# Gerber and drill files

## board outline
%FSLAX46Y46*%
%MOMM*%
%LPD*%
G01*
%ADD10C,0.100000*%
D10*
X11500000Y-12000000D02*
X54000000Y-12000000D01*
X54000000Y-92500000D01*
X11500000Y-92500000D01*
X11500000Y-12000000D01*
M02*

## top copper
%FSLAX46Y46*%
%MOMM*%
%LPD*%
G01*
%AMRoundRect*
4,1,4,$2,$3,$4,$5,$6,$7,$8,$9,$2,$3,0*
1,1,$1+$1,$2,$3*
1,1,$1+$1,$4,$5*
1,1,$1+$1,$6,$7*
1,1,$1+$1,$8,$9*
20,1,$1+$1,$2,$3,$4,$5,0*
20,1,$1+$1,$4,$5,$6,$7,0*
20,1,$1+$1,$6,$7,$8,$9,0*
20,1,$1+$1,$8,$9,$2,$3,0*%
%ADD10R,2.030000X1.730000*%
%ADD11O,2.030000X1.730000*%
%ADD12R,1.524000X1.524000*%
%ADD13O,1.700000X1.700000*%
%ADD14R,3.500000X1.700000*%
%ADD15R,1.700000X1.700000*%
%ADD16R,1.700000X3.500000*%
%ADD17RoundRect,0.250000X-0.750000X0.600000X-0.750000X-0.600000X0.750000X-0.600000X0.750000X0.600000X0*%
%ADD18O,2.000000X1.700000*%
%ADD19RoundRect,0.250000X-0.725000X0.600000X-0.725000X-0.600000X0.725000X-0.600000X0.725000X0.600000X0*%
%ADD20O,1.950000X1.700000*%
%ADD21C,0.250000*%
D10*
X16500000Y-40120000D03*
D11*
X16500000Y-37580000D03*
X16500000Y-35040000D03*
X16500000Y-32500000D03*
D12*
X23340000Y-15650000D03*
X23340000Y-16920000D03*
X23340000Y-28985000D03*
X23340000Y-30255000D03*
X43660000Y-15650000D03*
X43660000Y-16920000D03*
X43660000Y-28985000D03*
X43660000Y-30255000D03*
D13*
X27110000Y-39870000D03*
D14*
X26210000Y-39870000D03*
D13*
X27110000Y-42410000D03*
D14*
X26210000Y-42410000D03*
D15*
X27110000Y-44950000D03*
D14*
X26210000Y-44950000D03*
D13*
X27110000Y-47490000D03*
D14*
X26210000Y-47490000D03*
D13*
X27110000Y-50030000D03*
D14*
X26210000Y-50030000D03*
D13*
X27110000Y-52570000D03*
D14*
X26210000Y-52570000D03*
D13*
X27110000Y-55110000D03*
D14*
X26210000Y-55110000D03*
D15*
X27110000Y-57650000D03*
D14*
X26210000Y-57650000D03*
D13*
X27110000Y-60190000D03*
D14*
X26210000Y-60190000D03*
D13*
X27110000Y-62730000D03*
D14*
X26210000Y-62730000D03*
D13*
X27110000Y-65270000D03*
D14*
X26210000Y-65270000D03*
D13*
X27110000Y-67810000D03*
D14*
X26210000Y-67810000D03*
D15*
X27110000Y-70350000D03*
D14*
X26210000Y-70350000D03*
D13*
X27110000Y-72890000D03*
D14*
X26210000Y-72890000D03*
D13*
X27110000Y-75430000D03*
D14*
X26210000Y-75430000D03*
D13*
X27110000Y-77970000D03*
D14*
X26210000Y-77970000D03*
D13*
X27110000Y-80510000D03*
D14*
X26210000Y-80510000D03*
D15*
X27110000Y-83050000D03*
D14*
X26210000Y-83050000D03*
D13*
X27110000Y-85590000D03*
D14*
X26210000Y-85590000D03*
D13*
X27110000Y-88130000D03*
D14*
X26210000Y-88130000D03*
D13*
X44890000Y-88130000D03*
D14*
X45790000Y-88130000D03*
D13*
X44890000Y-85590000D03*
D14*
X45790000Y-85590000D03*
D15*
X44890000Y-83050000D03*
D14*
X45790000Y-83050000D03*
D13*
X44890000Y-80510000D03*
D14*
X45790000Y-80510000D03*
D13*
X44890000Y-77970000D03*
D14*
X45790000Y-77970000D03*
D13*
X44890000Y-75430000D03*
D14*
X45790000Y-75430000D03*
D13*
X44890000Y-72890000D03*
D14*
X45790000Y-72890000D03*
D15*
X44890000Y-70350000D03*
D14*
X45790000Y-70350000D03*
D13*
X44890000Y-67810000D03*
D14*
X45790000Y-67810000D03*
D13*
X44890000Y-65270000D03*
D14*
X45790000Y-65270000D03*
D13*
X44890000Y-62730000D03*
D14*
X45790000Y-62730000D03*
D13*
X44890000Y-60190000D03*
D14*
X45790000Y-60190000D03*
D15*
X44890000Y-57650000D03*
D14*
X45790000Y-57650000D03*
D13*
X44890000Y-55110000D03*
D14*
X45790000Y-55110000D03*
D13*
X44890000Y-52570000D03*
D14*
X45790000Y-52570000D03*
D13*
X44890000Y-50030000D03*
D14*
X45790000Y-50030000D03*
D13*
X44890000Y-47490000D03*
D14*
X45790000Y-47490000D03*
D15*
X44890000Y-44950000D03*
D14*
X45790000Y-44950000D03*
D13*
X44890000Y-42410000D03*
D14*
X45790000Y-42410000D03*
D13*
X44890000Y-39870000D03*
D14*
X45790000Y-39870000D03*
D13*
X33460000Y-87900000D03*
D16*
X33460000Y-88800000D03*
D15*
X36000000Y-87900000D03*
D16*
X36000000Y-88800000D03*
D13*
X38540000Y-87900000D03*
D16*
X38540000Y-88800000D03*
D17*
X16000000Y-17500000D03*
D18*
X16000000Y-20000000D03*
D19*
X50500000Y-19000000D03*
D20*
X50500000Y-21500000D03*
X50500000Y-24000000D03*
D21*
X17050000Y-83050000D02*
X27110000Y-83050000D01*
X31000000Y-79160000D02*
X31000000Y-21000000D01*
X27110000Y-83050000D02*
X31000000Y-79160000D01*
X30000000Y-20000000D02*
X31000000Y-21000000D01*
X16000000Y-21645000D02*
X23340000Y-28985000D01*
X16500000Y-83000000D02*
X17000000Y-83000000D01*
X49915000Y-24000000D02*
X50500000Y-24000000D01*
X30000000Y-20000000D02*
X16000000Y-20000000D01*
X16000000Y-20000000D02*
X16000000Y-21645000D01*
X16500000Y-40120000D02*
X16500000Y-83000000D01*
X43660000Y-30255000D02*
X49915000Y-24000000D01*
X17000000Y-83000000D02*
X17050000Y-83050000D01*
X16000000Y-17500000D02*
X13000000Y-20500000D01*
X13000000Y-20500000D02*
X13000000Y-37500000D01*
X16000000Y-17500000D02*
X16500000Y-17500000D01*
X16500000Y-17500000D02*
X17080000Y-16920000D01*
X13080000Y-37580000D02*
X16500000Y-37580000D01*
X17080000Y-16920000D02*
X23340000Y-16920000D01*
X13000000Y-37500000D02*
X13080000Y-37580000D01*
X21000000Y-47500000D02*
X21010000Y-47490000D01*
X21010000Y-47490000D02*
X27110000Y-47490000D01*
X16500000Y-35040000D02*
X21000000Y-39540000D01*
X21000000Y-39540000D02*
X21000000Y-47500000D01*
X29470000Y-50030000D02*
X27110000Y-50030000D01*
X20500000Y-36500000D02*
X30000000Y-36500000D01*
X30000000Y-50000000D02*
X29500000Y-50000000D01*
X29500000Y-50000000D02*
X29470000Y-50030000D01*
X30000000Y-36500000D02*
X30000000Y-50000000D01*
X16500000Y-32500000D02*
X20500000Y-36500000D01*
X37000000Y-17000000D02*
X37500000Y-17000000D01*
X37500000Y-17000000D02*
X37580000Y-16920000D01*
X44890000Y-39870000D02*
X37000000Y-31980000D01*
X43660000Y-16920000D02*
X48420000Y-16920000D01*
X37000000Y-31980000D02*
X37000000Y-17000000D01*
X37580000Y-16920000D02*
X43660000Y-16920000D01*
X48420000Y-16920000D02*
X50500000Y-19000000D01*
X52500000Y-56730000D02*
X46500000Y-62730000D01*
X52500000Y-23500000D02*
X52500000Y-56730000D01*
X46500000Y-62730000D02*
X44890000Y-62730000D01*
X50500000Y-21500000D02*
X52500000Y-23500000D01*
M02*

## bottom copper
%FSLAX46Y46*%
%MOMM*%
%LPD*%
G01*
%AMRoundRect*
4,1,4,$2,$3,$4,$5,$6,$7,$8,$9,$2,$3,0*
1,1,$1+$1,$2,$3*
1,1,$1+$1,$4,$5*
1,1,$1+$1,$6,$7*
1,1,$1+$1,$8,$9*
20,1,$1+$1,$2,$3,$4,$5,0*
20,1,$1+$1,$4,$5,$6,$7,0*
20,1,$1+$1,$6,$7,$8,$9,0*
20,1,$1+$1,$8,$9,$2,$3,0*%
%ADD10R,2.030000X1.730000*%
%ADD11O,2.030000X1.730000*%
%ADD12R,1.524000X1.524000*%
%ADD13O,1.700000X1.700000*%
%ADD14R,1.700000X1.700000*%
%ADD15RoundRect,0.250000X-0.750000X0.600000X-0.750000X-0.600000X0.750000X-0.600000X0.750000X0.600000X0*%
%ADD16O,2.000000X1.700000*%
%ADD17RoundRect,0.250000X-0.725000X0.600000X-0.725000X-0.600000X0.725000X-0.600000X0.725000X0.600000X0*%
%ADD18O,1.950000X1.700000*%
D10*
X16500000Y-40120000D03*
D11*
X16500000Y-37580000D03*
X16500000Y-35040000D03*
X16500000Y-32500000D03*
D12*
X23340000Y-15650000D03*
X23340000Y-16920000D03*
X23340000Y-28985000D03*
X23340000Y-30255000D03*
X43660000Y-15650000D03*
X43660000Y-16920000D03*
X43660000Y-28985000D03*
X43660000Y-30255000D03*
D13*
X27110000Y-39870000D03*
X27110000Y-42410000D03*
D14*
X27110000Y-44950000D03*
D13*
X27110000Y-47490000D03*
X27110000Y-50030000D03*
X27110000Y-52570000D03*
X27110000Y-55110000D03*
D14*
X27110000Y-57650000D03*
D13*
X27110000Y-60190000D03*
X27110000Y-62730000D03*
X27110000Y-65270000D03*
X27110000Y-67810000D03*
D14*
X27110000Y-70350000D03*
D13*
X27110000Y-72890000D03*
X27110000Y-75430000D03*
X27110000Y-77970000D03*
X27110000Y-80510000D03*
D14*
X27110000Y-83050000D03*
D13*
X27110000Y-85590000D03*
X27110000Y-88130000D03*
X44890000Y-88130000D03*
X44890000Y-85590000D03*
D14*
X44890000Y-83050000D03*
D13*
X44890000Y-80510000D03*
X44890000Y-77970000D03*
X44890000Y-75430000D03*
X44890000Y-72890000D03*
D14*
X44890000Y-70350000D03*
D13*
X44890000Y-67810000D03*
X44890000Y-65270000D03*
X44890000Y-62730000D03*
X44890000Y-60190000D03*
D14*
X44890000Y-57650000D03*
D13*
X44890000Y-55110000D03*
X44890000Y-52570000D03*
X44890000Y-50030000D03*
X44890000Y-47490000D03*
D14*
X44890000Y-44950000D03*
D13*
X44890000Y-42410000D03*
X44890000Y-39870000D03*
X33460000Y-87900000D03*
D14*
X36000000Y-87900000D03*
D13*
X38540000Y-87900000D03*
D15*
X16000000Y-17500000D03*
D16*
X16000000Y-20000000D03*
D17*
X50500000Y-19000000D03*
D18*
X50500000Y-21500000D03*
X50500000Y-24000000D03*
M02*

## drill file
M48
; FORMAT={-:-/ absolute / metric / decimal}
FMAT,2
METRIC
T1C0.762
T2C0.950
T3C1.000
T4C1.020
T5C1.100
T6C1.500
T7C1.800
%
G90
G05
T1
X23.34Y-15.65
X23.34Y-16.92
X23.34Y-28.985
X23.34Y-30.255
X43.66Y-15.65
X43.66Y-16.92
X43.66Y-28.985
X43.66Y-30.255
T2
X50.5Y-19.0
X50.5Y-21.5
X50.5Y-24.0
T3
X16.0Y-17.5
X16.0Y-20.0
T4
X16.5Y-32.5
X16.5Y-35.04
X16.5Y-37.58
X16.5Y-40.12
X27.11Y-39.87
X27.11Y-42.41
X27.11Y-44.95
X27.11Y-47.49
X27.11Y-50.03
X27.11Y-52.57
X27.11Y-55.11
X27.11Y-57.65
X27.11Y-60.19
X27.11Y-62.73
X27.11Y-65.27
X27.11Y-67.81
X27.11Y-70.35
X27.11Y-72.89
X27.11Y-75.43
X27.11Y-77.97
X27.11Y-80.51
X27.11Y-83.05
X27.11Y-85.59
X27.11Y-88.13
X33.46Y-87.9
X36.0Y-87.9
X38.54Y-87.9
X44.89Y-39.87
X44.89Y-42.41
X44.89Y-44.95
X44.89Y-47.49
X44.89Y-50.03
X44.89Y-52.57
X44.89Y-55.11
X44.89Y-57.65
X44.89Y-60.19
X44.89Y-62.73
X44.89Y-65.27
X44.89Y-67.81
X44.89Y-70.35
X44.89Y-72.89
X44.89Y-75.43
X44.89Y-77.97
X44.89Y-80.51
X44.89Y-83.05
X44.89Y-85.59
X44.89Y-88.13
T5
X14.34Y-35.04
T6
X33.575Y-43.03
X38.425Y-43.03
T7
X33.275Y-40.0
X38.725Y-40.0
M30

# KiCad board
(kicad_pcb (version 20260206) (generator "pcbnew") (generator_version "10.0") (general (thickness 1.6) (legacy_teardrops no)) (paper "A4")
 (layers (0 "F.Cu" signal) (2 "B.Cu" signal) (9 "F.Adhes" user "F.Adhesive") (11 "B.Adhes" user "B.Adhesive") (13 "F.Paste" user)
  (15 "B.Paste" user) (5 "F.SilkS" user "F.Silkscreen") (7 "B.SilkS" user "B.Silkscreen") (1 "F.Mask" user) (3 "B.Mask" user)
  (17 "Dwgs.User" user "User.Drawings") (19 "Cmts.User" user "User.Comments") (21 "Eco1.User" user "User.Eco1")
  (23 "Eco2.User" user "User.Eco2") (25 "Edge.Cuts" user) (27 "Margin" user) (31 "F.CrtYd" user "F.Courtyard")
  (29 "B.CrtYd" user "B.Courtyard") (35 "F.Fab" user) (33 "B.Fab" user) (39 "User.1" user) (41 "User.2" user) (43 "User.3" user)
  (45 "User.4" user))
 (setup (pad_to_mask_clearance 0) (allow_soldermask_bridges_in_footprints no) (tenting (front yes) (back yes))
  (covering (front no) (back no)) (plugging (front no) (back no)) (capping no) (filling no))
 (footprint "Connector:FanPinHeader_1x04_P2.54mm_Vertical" (layer "F.Cu") (at 16.5 40.12 90)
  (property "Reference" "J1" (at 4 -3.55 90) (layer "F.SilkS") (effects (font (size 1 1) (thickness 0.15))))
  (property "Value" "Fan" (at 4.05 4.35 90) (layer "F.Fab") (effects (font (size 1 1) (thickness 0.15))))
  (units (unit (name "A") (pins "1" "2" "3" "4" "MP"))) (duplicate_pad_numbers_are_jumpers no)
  (pad "" np_thru_hole circle (at 5.08 -2.16 180) (size 1.1 1.1) (drill 1.1) (layers "*.Cu" "*.Mask"))
  (pad "1" thru_hole rect (at 0 0 180) (size 2.03 1.73) (drill 1.02) (layers "*.Cu" "*.Mask") (remove_unused_layers no) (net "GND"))
  (pad "2" thru_hole oval (at 2.54 0 180) (size 2.03 1.73) (drill 1.02) (layers "*.Cu" "*.Mask") (remove_unused_layers no) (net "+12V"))
  (pad "3" thru_hole oval (at 5.08 0 180) (size 2.03 1.73) (drill 1.02) (layers "*.Cu" "*.Mask") (remove_unused_layers no)
   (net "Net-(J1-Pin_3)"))
  (pad "4" thru_hole oval (at 7.62 0 180) (size 2.03 1.73) (drill 1.02) (layers "*.Cu" "*.Mask") (remove_unused_layers no)
   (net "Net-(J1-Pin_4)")))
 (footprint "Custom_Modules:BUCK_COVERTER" (layer "F.Cu") (at 33.5 22)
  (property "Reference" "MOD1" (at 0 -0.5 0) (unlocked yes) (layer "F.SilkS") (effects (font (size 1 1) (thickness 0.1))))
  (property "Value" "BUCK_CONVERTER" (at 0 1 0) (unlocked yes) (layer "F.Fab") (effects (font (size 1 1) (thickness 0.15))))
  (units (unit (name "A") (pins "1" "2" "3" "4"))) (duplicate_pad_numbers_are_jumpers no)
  (pad "1" thru_hole rect (at -10.16 -6.35) (size 1.524 1.524) (drill 0.762) (layers "*.Cu" "*.Mask") (remove_unused_layers no) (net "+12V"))
  (pad "1" thru_hole rect (at -10.16 -5.08) (size 1.524 1.524) (drill 0.762) (layers "*.Cu" "*.Mask") (remove_unused_layers no) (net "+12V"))
  (pad "2" thru_hole rect (at -10.16 6.985) (size 1.524 1.524) (drill 0.762) (layers "*.Cu" "*.Mask") (remove_unused_layers no) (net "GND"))
  (pad "2" thru_hole rect (at -10.16 8.255) (size 1.524 1.524) (drill 0.762) (layers "*.Cu" "*.Mask") (remove_unused_layers no) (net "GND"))
  (pad "3" thru_hole rect (at 10.16 -6.35) (size 1.524 1.524) (drill 0.762) (layers "*.Cu" "*.Mask") (remove_unused_layers no) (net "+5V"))
  (pad "3" thru_hole rect (at 10.16 -5.08) (size 1.524 1.524) (drill 0.762) (layers "*.Cu" "*.Mask") (remove_unused_layers no) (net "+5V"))
  (pad "4" thru_hole rect (at 10.16 6.985) (size 1.524 1.524) (drill 0.762) (layers "*.Cu" "*.Mask") (remove_unused_layers no) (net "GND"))
  (pad "4" thru_hole rect (at 10.16 8.255) (size 1.524 1.524) (drill 0.762) (layers "*.Cu" "*.Mask") (remove_unused_layers no) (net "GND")))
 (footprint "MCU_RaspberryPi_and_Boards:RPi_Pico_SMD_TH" (layer "F.Cu") (at 36 64)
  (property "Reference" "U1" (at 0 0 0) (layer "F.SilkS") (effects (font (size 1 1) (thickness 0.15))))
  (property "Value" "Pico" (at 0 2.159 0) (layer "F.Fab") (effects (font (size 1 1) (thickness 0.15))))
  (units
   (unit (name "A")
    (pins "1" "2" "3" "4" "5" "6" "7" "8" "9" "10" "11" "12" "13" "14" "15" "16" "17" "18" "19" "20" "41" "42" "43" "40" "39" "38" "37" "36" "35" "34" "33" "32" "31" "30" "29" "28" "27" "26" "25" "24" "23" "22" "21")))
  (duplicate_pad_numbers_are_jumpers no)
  (pad "" np_thru_hole oval (at -2.725 -24) (size 1.8 1.8) (drill 1.8) (layers "*.Cu" "*.Mask"))
  (pad "" np_thru_hole oval (at -2.425 -20.97) (size 1.5 1.5) (drill 1.5) (layers "*.Cu" "*.Mask"))
  (pad "" np_thru_hole oval (at 2.425 -20.97) (size 1.5 1.5) (drill 1.5) (layers "*.Cu" "*.Mask"))
  (pad "" np_thru_hole oval (at 2.725 -24) (size 1.8 1.8) (drill 1.8) (layers "*.Cu" "*.Mask"))
  (pad "1" thru_hole oval (at -8.89 -24.13) (size 1.7 1.7) (drill 1.02) (layers "*.Cu" "*.Mask") (remove_unused_layers no)
   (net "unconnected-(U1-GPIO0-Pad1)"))
  (pad "1" smd rect (at -8.89 -24.13) (size 3.5 1.7) (drill (offset -0.9 0)) (layers "F.Cu" "F.Mask") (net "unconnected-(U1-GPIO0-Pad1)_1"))
  (pad "2" thru_hole oval (at -8.89 -21.59) (size 1.7 1.7) (drill 1.02) (layers "*.Cu" "*.Mask") (remove_unused_layers no)
   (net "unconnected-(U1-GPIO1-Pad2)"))
  (pad "2" smd rect (at -8.89 -21.59) (size 3.5 1.7) (drill (offset -0.9 0)) (layers "F.Cu" "F.Mask") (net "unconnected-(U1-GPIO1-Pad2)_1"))
  (pad "3" thru_hole rect (at -8.89 -19.05) (size 1.7 1.7) (drill 1.02) (layers "*.Cu" "*.Mask") (remove_unused_layers no) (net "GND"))
  (pad "3" smd rect (at -8.89 -19.05) (size 3.5 1.7) (drill (offset -0.9 0)) (layers "F.Cu" "F.Mask") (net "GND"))
  (pad "4" thru_hole oval (at -8.89 -16.51) (size 1.7 1.7) (drill 1.02) (layers "*.Cu" "*.Mask") (remove_unused_layers no)
   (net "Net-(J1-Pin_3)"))
  (pad "4" smd rect (at -8.89 -16.51) (size 3.5 1.7) (drill (offset -0.9 0)) (layers "F.Cu" "F.Mask") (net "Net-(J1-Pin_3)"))
  (pad "5" thru_hole oval (at -8.89 -13.97) (size 1.7 1.7) (drill 1.02) (layers "*.Cu" "*.Mask") (remove_unused_layers no)
   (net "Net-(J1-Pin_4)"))
  (pad "5" smd rect (at -8.89 -13.97) (size 3.5 1.7) (drill (offset -0.9 0)) (layers "F.Cu" "F.Mask") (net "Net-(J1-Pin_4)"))
  (pad "6" thru_hole oval (at -8.89 -11.43) (size 1.7 1.7) (drill 1.02) (layers "*.Cu" "*.Mask") (remove_unused_layers no)
   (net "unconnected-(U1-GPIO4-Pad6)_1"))
  (pad "6" smd rect (at -8.89 -11.43) (size 3.5 1.7) (drill (offset -0.9 0)) (layers "F.Cu" "F.Mask") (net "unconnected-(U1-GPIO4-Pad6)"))
  (pad "7" thru_hole oval (at -8.89 -8.89) (size 1.7 1.7) (drill 1.02) (layers "*.Cu" "*.Mask") (remove_unused_layers no)
   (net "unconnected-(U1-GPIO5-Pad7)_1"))
  (pad "7" smd rect (at -8.89 -8.89) (size 3.5 1.7) (drill (offset -0.9 0)) (layers "F.Cu" "F.Mask") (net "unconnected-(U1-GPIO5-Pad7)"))
  (pad "8" thru_hole rect (at -8.89 -6.35) (size 1.7 1.7) (drill 1.02) (layers "*.Cu" "*.Mask") (remove_unused_layers no)
   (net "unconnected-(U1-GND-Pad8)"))
  (pad "8" smd rect (at -8.89 -6.35) (size 3.5 1.7) (drill (offset -0.9 0)) (layers "F.Cu" "F.Mask") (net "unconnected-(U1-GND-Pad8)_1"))
  (pad "9" thru_hole oval (at -8.89 -3.81) (size 1.7 1.7) (drill 1.02) (layers "*.Cu" "*.Mask") (remove_unused_layers no)
   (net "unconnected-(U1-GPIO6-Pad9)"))
  (pad "9" smd rect (at -8.89 -3.81) (size 3.5 1.7) (drill (offset -0.9 0)) (layers "F.Cu" "F.Mask") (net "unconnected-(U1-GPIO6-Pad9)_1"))
  (pad "10" thru_hole oval (at -8.89 -1.27) (size 1.7 1.7) (drill 1.02) (layers "*.Cu" "*.Mask") (remove_unused_layers no)
   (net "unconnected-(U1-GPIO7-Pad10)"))
  (pad "10" smd rect (at -8.89 -1.27) (size 3.5 1.7) (drill (offset -0.9 0)) (layers "F.Cu" "F.Mask") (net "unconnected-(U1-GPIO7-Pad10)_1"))
  (pad "11" thru_hole oval (at -8.89 1.27) (size 1.7 1.7) (drill 1.02) (layers "*.Cu" "*.Mask") (remove_unused_layers no)
   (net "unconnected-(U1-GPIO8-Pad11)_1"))
  (pad "11" smd rect (at -8.89 1.27) (size 3.5 1.7) (drill (offset -0.9 0)) (layers "F.Cu" "F.Mask") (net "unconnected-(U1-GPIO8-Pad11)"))
  (pad "12" thru_hole oval (at -8.89 3.81) (size 1.7 1.7) (drill 1.02) (layers "*.Cu" "*.Mask") (remove_unused_layers no)
   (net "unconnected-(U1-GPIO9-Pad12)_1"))
  (pad "12" smd rect (at -8.89 3.81) (size 3.5 1.7) (drill (offset -0.9 0)) (layers "F.Cu" "F.Mask") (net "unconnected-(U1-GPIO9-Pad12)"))
  (pad "13" thru_hole rect (at -8.89 6.35) (size 1.7 1.7) (drill 1.02) (layers "*.Cu" "*.Mask") (remove_unused_layers no)
   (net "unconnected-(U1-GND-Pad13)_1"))
  (pad "13" smd rect (at -8.89 6.35) (size 3.5 1.7) (drill (offset -0.9 0)) (layers "F.Cu" "F.Mask") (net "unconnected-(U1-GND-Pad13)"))
  (pad "14" thru_hole oval (at -8.89 8.89) (size 1.7 1.7) (drill 1.02) (layers "*.Cu" "*.Mask") (remove_unused_layers no)
   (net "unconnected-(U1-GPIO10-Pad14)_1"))
  (pad "14" smd rect (at -8.89 8.89) (size 3.5 1.7) (drill (offset -0.9 0)) (layers "F.Cu" "F.Mask") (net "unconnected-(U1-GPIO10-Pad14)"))
  (pad "15" thru_hole oval (at -8.89 11.43) (size 1.7 1.7) (drill 1.02) (layers "*.Cu" "*.Mask") (remove_unused_layers no)
   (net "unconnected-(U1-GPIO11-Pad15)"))
  (pad "15" smd rect (at -8.89 11.43) (size 3.5 1.7) (drill (offset -0.9 0)) (layers "F.Cu" "F.Mask")
   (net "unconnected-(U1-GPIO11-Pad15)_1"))
  (pad "16" thru_hole oval (at -8.89 13.97) (size 1.7 1.7) (drill 1.02) (layers "*.Cu" "*.Mask") (remove_unused_layers no)
   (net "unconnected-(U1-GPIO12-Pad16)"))
  (pad "16" smd rect (at -8.89 13.97) (size 3.5 1.7) (drill (offset -0.9 0)) (layers "F.Cu" "F.Mask")
   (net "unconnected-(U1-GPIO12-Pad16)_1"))
  (pad "17" thru_hole oval (at -8.89 16.51) (size 1.7 1.7) (drill 1.02) (layers "*.Cu" "*.Mask") (remove_unused_layers no)
   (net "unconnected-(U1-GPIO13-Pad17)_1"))
  (pad "17" smd rect (at -8.89 16.51) (size 3.5 1.7) (drill (offset -0.9 0)) (layers "F.Cu" "F.Mask") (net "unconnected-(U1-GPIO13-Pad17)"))
  (pad "18" thru_hole rect (at -8.89 19.05) (size 1.7 1.7) (drill 1.02) (layers "*.Cu" "*.Mask") (remove_unused_layers no) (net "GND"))
  (pad "18" smd rect (at -8.89 19.05) (size 3.5 1.7) (drill (offset -0.9 0)) (layers "F.Cu" "F.Mask") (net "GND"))
  (pad "19" thru_hole oval (at -8.89 21.59) (size 1.7 1.7) (drill 1.02) (layers "*.Cu" "*.Mask") (remove_unused_layers no)
   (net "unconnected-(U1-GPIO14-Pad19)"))
  (pad "19" smd rect (at -8.89 21.59) (size 3.5 1.7) (drill (offset -0.9 0)) (layers "F.Cu" "F.Mask")
   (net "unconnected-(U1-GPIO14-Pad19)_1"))
  (pad "20" thru_hole oval (at -8.89 24.13) (size 1.7 1.7) (drill 1.02) (layers "*.Cu" "*.Mask") (remove_unused_layers no)
   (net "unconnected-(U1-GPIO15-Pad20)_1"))
  (pad "20" smd rect (at -8.89 24.13) (size 3.5 1.7) (drill (offset -0.9 0)) (layers "F.Cu" "F.Mask") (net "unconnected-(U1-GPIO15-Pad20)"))
  (pad "21" thru_hole oval (at 8.89 24.13) (size 1.7 1.7) (drill 1.02) (layers "*.Cu" "*.Mask") (remove_unused_layers no)
   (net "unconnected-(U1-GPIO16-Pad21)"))
  (pad "21" smd rect (at 8.89 24.13) (size 3.5 1.7) (drill (offset 0.9 0)) (layers "F.Cu" "F.Mask") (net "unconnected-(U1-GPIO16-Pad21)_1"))
  (pad "22" thru_hole oval (at 8.89 21.59) (size 1.7 1.7) (drill 1.02) (layers "*.Cu" "*.Mask") (remove_unused_layers no)
   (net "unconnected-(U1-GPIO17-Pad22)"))
  (pad "22" smd rect (at 8.89 21.59) (size 3.5 1.7) (drill (offset 0.9 0)) (layers "F.Cu" "F.Mask") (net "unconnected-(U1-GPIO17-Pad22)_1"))
  (pad "23" thru_hole rect (at 8.89 19.05) (size 1.7 1.7) (drill 1.02) (layers "*.Cu" "*.Mask") (remove_unused_layers no)
   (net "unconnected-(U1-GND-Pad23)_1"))
  (pad "23" smd rect (at 8.89 19.05) (size 3.5 1.7) (drill (offset 0.9 0)) (layers "F.Cu" "F.Mask") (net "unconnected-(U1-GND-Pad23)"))
  (pad "24" thru_hole oval (at 8.89 16.51) (size 1.7 1.7) (drill 1.02) (layers "*.Cu" "*.Mask") (remove_unused_layers no)
   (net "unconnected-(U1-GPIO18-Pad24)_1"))
  (pad "24" smd rect (at 8.89 16.51) (size 3.5 1.7) (drill (offset 0.9 0)) (layers "F.Cu" "F.Mask") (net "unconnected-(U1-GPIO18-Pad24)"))
  (pad "25" thru_hole oval (at 8.89 13.97) (size 1.7 1.7) (drill 1.02) (layers "*.Cu" "*.Mask") (remove_unused_layers no)
   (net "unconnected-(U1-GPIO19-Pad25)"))
  (pad "25" smd rect (at 8.89 13.97) (size 3.5 1.7) (drill (offset 0.9 0)) (layers "F.Cu" "F.Mask") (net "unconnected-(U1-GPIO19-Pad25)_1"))
  (pad "26" thru_hole oval (at 8.89 11.43) (size 1.7 1.7) (drill 1.02) (layers "*.Cu" "*.Mask") (remove_unused_layers no)
   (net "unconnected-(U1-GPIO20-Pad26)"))
  (pad "26" smd rect (at 8.89 11.43) (size 3.5 1.7) (drill (offset 0.9 0)) (layers "F.Cu" "F.Mask") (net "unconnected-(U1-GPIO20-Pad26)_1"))
  (pad "27" thru_hole oval (at 8.89 8.89) (size 1.7 1.7) (drill 1.02) (layers "*.Cu" "*.Mask") (remove_unused_layers no)
   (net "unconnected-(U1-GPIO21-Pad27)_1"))
  (pad "27" smd rect (at 8.89 8.89) (size 3.5 1.7) (drill (offset 0.9 0)) (layers "F.Cu" "F.Mask") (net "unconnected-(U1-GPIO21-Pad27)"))
  (pad "28" thru_hole rect (at 8.89 6.35) (size 1.7 1.7) (drill 1.02) (layers "*.Cu" "*.Mask") (remove_unused_layers no)
   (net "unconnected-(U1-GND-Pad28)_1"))
  (pad "28" smd rect (at 8.89 6.35) (size 3.5 1.7) (drill (offset 0.9 0)) (layers "F.Cu" "F.Mask") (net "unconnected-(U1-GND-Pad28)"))
  (pad "29" thru_hole oval (at 8.89 3.81) (size 1.7 1.7) (drill 1.02) (layers "*.Cu" "*.Mask") (remove_unused_layers no)
   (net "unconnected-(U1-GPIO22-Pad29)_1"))
  (pad "29" smd rect (at 8.89 3.81) (size 3.5 1.7) (drill (offset 0.9 0)) (layers "F.Cu" "F.Mask") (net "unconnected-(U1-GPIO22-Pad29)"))
  (pad "30" thru_hole oval (at 8.89 1.27) (size 1.7 1.7) (drill 1.02) (layers "*.Cu" "*.Mask") (remove_unused_layers no)
   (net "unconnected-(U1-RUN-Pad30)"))
  (pad "30" smd rect (at 8.89 1.27) (size 3.5 1.7) (drill (offset 0.9 0)) (layers "F.Cu" "F.Mask") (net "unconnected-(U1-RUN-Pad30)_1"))
  (pad "31" thru_hole oval (at 8.89 -1.27) (size 1.7 1.7) (drill 1.02) (layers "*.Cu" "*.Mask") (remove_unused_layers no)
   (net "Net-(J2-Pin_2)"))
  (pad "31" smd rect (at 8.89 -1.27) (size 3.5 1.7) (drill (offset 0.9 0)) (layers "F.Cu" "F.Mask") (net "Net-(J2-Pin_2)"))
  (pad "32" thru_hole oval (at 8.89 -3.81) (size 1.7 1.7) (drill 1.02) (layers "*.Cu" "*.Mask") (remove_unused_layers no)
   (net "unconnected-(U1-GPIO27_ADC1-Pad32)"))
  (pad "32" smd rect (at 8.89 -3.81) (size 3.5 1.7) (drill (offset 0.9 0)) (layers "F.Cu" "F.Mask")
   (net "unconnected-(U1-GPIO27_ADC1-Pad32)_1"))
  (pad "33" thru_hole rect (at 8.89 -6.35) (size 1.7 1.7) (drill 1.02) (layers "*.Cu" "*.Mask") (remove_unused_layers no)
   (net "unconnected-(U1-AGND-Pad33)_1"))
  (pad "33" smd rect (at 8.89 -6.35) (size 3.5 1.7) (drill (offset 0.9 0)) (layers "F.Cu" "F.Mask") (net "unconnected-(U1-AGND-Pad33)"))
  (pad "34" thru_hole oval (at 8.89 -8.89) (size 1.7 1.7) (drill 1.02) (layers "*.Cu" "*.Mask") (remove_unused_layers no)
   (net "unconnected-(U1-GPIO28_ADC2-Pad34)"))
  (pad "34" smd rect (at 8.89 -8.89) (size 3.5 1.7) (drill (offset 0.9 0)) (layers "F.Cu" "F.Mask")
   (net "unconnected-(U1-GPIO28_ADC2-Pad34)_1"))
  (pad "35" thru_hole oval (at 8.89 -11.43) (size 1.7 1.7) (drill 1.02) (layers "*.Cu" "*.Mask") (remove_unused_layers no)
   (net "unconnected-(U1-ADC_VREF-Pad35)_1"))
  (pad "35" smd rect (at 8.89 -11.43) (size 3.5 1.7) (drill (offset 0.9 0)) (layers "F.Cu" "F.Mask") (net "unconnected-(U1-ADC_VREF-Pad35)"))
  (pad "36" thru_hole oval (at 8.89 -13.97) (size 1.7 1.7) (drill 1.02) (layers "*.Cu" "*.Mask") (remove_unused_layers no)
   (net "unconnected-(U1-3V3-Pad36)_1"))
  (pad "36" smd rect (at 8.89 -13.97) (size 3.5 1.7) (drill (offset 0.9 0)) (layers "F.Cu" "F.Mask") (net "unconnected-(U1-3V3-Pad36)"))
  (pad "37" thru_hole oval (at 8.89 -16.51) (size 1.7 1.7) (drill 1.02) (layers "*.Cu" "*.Mask") (remove_unused_layers no)
   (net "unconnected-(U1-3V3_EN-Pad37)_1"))
  (pad "37" smd rect (at 8.89 -16.51) (size 3.5 1.7) (drill (offset 0.9 0)) (layers "F.Cu" "F.Mask") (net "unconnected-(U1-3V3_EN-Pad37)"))
  (pad "38" thru_hole rect (at 8.89 -19.05) (size 1.7 1.7) (drill 1.02) (layers "*.Cu" "*.Mask") (remove_unused_layers no)
   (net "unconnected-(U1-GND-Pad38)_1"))
  (pad "38" smd rect (at 8.89 -19.05) (size 3.5 1.7) (drill (offset 0.9 0)) (layers "F.Cu" "F.Mask") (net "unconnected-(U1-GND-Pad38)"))
  (pad "39" thru_hole oval (at 8.89 -21.59) (size 1.7 1.7) (drill 1.02) (layers "*.Cu" "*.Mask") (remove_unused_layers no)
   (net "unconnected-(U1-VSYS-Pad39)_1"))
  (pad "39" smd rect (at 8.89 -21.59) (size 3.5 1.7) (drill (offset 0.9 0)) (layers "F.Cu" "F.Mask") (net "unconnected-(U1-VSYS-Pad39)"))
  (pad "40" thru_hole oval (at 8.89 -24.13) (size 1.7 1.7) (drill 1.02) (layers "*.Cu" "*.Mask") (remove_unused_layers no) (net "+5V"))
  (pad "40" smd rect (at 8.89 -24.13) (size 3.5 1.7) (drill (offset 0.9 0)) (layers "F.Cu" "F.Mask") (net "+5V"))
  (pad "41" thru_hole oval (at -2.54 23.9) (size 1.7 1.7) (drill 1.02) (layers "*.Cu" "*.Mask") (remove_unused_layers no)
   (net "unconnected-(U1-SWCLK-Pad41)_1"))
  (pad "41" smd rect (at -2.54 23.9 90) (size 3.5 1.7) (drill (offset -0.9 0)) (layers "F.Cu" "F.Mask") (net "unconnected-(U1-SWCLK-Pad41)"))
  (pad "42" thru_hole rect (at 0 23.9) (size 1.7 1.7) (drill 1.02) (layers "*.Cu" "*.Mask") (remove_unused_layers no)
   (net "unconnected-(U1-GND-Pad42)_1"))
  (pad "42" smd rect (at 0 23.9 90) (size 3.5 1.7) (drill (offset -0.9 0)) (layers "F.Cu" "F.Mask") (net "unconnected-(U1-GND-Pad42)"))
  (pad "43" thru_hole oval (at 2.54 23.9) (size 1.7 1.7) (drill 1.02) (layers "*.Cu" "*.Mask") (remove_unused_layers no)
   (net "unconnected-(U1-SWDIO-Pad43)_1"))
  (pad "43" smd rect (at 2.54 23.9 90) (size 3.5 1.7) (drill (offset -0.9 0)) (layers "F.Cu" "F.Mask") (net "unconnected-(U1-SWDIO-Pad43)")))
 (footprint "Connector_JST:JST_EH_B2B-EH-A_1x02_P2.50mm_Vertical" (layer "F.Cu") (at 16 17.5 -90)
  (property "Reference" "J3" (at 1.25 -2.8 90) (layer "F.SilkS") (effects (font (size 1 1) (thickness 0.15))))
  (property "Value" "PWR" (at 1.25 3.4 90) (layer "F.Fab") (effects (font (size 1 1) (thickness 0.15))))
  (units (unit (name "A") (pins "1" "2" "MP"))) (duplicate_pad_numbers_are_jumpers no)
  (pad "1" thru_hole roundrect (at 0 0 270) (size 1.7 2) (drill 1) (layers "*.Cu" "*.Mask") (remove_unused_layers no)
   (roundrect_rratio 0.147059) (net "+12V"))
  (pad "2" thru_hole oval (at 2.5 0 270) (size 1.7 2) (drill 1) (layers "*.Cu" "*.Mask") (remove_unused_layers no) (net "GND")))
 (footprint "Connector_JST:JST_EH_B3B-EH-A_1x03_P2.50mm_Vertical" (layer "F.Cu") (at 50.5 19 -90)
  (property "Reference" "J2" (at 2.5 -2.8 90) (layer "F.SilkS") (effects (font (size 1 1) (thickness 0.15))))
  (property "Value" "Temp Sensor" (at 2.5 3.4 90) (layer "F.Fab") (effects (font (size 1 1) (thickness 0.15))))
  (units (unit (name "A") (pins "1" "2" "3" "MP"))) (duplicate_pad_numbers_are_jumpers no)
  (pad "1" thru_hole roundrect (at 0 0 270) (size 1.7 1.95) (drill 0.95) (layers "*.Cu" "*.Mask") (remove_unused_layers no)
   (roundrect_rratio 0.147059) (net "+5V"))
  (pad "2" thru_hole oval (at 2.5 0 270) (size 1.7 1.95) (drill 0.95) (layers "*.Cu" "*.Mask") (remove_unused_layers no)
   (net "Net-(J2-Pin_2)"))
  (pad "3" thru_hole oval (at 5 0 270) (size 1.7 1.95) (drill 0.95) (layers "*.Cu" "*.Mask") (remove_unused_layers no) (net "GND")))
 (gr_rect (start 11.5 12) (end 54 92.5) (stroke (width 0.1) (type default)) (fill no) (layer "Edge.Cuts"))
 (segment (start 17.05 83.05) (end 27.11 83.05) (width 0.25) (layer "F.Cu") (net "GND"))
 (segment (start 31 79.16) (end 31 21) (width 0.25) (layer "F.Cu") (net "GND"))
 (segment (start 27.11 83.05) (end 31 79.16) (width 0.25) (layer "F.Cu") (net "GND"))
 (segment (start 30 20) (end 31 21) (width 0.25) (layer "F.Cu") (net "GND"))
 (segment (start 16 21.645) (end 23.34 28.985) (width 0.25) (layer "F.Cu") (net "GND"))
 (segment (start 16.5 83) (end 17 83) (width 0.25) (layer "F.Cu") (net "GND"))
 (segment (start 49.915 24) (end 50.5 24) (width 0.25) (layer "F.Cu") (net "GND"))
 (segment (start 30 20) (end 16 20) (width 0.25) (layer "F.Cu") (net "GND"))
 (segment (start 16 20) (end 16 21.645) (width 0.25) (layer "F.Cu") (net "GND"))
 (segment (start 16.5 40.12) (end 16.5 83) (width 0.25) (layer "F.Cu") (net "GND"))
 (segment (start 43.66 30.255) (end 49.915 24) (width 0.25) (layer "F.Cu") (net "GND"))
 (segment (start 17 83) (end 17.05 83.05) (width 0.25) (layer "F.Cu") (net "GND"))
 (segment (start 16 17.5) (end 13 20.5) (width 0.25) (layer "F.Cu") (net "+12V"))
 (segment (start 13 20.5) (end 13 37.5) (width 0.25) (layer "F.Cu") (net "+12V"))
 (segment (start 16 17.5) (end 16.5 17.5) (width 0.25) (layer "F.Cu") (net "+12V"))
 (segment (start 16.5 17.5) (end 17.08 16.92) (width 0.25) (layer "F.Cu") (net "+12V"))
 (segment (start 13.08 37.58) (end 16.5 37.58) (width 0.25) (layer "F.Cu") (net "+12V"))
 (segment (start 17.08 16.92) (end 23.34 16.92) (width 0.25) (layer "F.Cu") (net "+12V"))
 (segment (start 13 37.5) (end 13.08 37.58) (width 0.25) (layer "F.Cu") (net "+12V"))
 (segment (start 21 47.5) (end 21.01 47.49) (width 0.25) (layer "F.Cu") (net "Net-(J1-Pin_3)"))
 (segment (start 21.01 47.49) (end 27.11 47.49) (width 0.25) (layer "F.Cu") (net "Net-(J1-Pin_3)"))
 (segment (start 16.5 35.04) (end 21 39.54) (width 0.25) (layer "F.Cu") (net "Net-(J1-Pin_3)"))
 (segment (start 21 39.54) (end 21 47.5) (width 0.25) (layer "F.Cu") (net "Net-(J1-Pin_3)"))
 (segment (start 29.47 50.03) (end 27.11 50.03) (width 0.25) (layer "F.Cu") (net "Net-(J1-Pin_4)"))
 (segment (start 20.5 36.5) (end 30 36.5) (width 0.25) (layer "F.Cu") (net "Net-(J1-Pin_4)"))
 (segment (start 30 50) (end 29.5 50) (width 0.25) (layer "F.Cu") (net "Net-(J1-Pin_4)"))
 (segment (start 29.5 50) (end 29.47 50.03) (width 0.25) (layer "F.Cu") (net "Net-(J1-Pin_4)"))
 (segment (start 30 36.5) (end 30 50) (width 0.25) (layer "F.Cu") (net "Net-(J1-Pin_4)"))
 (segment (start 16.5 32.5) (end 20.5 36.5) (width 0.25) (layer "F.Cu") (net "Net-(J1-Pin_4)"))
 (segment (start 37 17) (end 37.5 17) (width 0.25) (layer "F.Cu") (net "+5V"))
 (segment (start 37.5 17) (end 37.58 16.92) (width 0.25) (layer "F.Cu") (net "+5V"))
 (segment (start 44.89 39.87) (end 37 31.98) (width 0.25) (layer "F.Cu") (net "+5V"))
 (segment (start 43.66 16.92) (end 48.42 16.92) (width 0.25) (layer "F.Cu") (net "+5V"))
 (segment (start 37 31.98) (end 37 17) (width 0.25) (layer "F.Cu") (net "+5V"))
 (segment (start 37.58 16.92) (end 43.66 16.92) (width 0.25) (layer "F.Cu") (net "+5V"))
 (segment (start 48.42 16.92) (end 50.5 19) (width 0.25) (layer "F.Cu") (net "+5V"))
 (segment (start 52.5 56.73) (end 46.5 62.73) (width 0.25) (layer "F.Cu") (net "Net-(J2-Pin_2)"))
 (segment (start 52.5 23.5) (end 52.5 56.73) (width 0.25) (layer "F.Cu") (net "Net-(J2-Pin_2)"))
 (segment (start 46.5 62.73) (end 44.89 62.73) (width 0.25) (layer "F.Cu") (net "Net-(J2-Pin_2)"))
 (segment (start 50.5 21.5) (end 52.5 23.5) (width 0.25) (layer "F.Cu") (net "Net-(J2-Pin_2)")))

